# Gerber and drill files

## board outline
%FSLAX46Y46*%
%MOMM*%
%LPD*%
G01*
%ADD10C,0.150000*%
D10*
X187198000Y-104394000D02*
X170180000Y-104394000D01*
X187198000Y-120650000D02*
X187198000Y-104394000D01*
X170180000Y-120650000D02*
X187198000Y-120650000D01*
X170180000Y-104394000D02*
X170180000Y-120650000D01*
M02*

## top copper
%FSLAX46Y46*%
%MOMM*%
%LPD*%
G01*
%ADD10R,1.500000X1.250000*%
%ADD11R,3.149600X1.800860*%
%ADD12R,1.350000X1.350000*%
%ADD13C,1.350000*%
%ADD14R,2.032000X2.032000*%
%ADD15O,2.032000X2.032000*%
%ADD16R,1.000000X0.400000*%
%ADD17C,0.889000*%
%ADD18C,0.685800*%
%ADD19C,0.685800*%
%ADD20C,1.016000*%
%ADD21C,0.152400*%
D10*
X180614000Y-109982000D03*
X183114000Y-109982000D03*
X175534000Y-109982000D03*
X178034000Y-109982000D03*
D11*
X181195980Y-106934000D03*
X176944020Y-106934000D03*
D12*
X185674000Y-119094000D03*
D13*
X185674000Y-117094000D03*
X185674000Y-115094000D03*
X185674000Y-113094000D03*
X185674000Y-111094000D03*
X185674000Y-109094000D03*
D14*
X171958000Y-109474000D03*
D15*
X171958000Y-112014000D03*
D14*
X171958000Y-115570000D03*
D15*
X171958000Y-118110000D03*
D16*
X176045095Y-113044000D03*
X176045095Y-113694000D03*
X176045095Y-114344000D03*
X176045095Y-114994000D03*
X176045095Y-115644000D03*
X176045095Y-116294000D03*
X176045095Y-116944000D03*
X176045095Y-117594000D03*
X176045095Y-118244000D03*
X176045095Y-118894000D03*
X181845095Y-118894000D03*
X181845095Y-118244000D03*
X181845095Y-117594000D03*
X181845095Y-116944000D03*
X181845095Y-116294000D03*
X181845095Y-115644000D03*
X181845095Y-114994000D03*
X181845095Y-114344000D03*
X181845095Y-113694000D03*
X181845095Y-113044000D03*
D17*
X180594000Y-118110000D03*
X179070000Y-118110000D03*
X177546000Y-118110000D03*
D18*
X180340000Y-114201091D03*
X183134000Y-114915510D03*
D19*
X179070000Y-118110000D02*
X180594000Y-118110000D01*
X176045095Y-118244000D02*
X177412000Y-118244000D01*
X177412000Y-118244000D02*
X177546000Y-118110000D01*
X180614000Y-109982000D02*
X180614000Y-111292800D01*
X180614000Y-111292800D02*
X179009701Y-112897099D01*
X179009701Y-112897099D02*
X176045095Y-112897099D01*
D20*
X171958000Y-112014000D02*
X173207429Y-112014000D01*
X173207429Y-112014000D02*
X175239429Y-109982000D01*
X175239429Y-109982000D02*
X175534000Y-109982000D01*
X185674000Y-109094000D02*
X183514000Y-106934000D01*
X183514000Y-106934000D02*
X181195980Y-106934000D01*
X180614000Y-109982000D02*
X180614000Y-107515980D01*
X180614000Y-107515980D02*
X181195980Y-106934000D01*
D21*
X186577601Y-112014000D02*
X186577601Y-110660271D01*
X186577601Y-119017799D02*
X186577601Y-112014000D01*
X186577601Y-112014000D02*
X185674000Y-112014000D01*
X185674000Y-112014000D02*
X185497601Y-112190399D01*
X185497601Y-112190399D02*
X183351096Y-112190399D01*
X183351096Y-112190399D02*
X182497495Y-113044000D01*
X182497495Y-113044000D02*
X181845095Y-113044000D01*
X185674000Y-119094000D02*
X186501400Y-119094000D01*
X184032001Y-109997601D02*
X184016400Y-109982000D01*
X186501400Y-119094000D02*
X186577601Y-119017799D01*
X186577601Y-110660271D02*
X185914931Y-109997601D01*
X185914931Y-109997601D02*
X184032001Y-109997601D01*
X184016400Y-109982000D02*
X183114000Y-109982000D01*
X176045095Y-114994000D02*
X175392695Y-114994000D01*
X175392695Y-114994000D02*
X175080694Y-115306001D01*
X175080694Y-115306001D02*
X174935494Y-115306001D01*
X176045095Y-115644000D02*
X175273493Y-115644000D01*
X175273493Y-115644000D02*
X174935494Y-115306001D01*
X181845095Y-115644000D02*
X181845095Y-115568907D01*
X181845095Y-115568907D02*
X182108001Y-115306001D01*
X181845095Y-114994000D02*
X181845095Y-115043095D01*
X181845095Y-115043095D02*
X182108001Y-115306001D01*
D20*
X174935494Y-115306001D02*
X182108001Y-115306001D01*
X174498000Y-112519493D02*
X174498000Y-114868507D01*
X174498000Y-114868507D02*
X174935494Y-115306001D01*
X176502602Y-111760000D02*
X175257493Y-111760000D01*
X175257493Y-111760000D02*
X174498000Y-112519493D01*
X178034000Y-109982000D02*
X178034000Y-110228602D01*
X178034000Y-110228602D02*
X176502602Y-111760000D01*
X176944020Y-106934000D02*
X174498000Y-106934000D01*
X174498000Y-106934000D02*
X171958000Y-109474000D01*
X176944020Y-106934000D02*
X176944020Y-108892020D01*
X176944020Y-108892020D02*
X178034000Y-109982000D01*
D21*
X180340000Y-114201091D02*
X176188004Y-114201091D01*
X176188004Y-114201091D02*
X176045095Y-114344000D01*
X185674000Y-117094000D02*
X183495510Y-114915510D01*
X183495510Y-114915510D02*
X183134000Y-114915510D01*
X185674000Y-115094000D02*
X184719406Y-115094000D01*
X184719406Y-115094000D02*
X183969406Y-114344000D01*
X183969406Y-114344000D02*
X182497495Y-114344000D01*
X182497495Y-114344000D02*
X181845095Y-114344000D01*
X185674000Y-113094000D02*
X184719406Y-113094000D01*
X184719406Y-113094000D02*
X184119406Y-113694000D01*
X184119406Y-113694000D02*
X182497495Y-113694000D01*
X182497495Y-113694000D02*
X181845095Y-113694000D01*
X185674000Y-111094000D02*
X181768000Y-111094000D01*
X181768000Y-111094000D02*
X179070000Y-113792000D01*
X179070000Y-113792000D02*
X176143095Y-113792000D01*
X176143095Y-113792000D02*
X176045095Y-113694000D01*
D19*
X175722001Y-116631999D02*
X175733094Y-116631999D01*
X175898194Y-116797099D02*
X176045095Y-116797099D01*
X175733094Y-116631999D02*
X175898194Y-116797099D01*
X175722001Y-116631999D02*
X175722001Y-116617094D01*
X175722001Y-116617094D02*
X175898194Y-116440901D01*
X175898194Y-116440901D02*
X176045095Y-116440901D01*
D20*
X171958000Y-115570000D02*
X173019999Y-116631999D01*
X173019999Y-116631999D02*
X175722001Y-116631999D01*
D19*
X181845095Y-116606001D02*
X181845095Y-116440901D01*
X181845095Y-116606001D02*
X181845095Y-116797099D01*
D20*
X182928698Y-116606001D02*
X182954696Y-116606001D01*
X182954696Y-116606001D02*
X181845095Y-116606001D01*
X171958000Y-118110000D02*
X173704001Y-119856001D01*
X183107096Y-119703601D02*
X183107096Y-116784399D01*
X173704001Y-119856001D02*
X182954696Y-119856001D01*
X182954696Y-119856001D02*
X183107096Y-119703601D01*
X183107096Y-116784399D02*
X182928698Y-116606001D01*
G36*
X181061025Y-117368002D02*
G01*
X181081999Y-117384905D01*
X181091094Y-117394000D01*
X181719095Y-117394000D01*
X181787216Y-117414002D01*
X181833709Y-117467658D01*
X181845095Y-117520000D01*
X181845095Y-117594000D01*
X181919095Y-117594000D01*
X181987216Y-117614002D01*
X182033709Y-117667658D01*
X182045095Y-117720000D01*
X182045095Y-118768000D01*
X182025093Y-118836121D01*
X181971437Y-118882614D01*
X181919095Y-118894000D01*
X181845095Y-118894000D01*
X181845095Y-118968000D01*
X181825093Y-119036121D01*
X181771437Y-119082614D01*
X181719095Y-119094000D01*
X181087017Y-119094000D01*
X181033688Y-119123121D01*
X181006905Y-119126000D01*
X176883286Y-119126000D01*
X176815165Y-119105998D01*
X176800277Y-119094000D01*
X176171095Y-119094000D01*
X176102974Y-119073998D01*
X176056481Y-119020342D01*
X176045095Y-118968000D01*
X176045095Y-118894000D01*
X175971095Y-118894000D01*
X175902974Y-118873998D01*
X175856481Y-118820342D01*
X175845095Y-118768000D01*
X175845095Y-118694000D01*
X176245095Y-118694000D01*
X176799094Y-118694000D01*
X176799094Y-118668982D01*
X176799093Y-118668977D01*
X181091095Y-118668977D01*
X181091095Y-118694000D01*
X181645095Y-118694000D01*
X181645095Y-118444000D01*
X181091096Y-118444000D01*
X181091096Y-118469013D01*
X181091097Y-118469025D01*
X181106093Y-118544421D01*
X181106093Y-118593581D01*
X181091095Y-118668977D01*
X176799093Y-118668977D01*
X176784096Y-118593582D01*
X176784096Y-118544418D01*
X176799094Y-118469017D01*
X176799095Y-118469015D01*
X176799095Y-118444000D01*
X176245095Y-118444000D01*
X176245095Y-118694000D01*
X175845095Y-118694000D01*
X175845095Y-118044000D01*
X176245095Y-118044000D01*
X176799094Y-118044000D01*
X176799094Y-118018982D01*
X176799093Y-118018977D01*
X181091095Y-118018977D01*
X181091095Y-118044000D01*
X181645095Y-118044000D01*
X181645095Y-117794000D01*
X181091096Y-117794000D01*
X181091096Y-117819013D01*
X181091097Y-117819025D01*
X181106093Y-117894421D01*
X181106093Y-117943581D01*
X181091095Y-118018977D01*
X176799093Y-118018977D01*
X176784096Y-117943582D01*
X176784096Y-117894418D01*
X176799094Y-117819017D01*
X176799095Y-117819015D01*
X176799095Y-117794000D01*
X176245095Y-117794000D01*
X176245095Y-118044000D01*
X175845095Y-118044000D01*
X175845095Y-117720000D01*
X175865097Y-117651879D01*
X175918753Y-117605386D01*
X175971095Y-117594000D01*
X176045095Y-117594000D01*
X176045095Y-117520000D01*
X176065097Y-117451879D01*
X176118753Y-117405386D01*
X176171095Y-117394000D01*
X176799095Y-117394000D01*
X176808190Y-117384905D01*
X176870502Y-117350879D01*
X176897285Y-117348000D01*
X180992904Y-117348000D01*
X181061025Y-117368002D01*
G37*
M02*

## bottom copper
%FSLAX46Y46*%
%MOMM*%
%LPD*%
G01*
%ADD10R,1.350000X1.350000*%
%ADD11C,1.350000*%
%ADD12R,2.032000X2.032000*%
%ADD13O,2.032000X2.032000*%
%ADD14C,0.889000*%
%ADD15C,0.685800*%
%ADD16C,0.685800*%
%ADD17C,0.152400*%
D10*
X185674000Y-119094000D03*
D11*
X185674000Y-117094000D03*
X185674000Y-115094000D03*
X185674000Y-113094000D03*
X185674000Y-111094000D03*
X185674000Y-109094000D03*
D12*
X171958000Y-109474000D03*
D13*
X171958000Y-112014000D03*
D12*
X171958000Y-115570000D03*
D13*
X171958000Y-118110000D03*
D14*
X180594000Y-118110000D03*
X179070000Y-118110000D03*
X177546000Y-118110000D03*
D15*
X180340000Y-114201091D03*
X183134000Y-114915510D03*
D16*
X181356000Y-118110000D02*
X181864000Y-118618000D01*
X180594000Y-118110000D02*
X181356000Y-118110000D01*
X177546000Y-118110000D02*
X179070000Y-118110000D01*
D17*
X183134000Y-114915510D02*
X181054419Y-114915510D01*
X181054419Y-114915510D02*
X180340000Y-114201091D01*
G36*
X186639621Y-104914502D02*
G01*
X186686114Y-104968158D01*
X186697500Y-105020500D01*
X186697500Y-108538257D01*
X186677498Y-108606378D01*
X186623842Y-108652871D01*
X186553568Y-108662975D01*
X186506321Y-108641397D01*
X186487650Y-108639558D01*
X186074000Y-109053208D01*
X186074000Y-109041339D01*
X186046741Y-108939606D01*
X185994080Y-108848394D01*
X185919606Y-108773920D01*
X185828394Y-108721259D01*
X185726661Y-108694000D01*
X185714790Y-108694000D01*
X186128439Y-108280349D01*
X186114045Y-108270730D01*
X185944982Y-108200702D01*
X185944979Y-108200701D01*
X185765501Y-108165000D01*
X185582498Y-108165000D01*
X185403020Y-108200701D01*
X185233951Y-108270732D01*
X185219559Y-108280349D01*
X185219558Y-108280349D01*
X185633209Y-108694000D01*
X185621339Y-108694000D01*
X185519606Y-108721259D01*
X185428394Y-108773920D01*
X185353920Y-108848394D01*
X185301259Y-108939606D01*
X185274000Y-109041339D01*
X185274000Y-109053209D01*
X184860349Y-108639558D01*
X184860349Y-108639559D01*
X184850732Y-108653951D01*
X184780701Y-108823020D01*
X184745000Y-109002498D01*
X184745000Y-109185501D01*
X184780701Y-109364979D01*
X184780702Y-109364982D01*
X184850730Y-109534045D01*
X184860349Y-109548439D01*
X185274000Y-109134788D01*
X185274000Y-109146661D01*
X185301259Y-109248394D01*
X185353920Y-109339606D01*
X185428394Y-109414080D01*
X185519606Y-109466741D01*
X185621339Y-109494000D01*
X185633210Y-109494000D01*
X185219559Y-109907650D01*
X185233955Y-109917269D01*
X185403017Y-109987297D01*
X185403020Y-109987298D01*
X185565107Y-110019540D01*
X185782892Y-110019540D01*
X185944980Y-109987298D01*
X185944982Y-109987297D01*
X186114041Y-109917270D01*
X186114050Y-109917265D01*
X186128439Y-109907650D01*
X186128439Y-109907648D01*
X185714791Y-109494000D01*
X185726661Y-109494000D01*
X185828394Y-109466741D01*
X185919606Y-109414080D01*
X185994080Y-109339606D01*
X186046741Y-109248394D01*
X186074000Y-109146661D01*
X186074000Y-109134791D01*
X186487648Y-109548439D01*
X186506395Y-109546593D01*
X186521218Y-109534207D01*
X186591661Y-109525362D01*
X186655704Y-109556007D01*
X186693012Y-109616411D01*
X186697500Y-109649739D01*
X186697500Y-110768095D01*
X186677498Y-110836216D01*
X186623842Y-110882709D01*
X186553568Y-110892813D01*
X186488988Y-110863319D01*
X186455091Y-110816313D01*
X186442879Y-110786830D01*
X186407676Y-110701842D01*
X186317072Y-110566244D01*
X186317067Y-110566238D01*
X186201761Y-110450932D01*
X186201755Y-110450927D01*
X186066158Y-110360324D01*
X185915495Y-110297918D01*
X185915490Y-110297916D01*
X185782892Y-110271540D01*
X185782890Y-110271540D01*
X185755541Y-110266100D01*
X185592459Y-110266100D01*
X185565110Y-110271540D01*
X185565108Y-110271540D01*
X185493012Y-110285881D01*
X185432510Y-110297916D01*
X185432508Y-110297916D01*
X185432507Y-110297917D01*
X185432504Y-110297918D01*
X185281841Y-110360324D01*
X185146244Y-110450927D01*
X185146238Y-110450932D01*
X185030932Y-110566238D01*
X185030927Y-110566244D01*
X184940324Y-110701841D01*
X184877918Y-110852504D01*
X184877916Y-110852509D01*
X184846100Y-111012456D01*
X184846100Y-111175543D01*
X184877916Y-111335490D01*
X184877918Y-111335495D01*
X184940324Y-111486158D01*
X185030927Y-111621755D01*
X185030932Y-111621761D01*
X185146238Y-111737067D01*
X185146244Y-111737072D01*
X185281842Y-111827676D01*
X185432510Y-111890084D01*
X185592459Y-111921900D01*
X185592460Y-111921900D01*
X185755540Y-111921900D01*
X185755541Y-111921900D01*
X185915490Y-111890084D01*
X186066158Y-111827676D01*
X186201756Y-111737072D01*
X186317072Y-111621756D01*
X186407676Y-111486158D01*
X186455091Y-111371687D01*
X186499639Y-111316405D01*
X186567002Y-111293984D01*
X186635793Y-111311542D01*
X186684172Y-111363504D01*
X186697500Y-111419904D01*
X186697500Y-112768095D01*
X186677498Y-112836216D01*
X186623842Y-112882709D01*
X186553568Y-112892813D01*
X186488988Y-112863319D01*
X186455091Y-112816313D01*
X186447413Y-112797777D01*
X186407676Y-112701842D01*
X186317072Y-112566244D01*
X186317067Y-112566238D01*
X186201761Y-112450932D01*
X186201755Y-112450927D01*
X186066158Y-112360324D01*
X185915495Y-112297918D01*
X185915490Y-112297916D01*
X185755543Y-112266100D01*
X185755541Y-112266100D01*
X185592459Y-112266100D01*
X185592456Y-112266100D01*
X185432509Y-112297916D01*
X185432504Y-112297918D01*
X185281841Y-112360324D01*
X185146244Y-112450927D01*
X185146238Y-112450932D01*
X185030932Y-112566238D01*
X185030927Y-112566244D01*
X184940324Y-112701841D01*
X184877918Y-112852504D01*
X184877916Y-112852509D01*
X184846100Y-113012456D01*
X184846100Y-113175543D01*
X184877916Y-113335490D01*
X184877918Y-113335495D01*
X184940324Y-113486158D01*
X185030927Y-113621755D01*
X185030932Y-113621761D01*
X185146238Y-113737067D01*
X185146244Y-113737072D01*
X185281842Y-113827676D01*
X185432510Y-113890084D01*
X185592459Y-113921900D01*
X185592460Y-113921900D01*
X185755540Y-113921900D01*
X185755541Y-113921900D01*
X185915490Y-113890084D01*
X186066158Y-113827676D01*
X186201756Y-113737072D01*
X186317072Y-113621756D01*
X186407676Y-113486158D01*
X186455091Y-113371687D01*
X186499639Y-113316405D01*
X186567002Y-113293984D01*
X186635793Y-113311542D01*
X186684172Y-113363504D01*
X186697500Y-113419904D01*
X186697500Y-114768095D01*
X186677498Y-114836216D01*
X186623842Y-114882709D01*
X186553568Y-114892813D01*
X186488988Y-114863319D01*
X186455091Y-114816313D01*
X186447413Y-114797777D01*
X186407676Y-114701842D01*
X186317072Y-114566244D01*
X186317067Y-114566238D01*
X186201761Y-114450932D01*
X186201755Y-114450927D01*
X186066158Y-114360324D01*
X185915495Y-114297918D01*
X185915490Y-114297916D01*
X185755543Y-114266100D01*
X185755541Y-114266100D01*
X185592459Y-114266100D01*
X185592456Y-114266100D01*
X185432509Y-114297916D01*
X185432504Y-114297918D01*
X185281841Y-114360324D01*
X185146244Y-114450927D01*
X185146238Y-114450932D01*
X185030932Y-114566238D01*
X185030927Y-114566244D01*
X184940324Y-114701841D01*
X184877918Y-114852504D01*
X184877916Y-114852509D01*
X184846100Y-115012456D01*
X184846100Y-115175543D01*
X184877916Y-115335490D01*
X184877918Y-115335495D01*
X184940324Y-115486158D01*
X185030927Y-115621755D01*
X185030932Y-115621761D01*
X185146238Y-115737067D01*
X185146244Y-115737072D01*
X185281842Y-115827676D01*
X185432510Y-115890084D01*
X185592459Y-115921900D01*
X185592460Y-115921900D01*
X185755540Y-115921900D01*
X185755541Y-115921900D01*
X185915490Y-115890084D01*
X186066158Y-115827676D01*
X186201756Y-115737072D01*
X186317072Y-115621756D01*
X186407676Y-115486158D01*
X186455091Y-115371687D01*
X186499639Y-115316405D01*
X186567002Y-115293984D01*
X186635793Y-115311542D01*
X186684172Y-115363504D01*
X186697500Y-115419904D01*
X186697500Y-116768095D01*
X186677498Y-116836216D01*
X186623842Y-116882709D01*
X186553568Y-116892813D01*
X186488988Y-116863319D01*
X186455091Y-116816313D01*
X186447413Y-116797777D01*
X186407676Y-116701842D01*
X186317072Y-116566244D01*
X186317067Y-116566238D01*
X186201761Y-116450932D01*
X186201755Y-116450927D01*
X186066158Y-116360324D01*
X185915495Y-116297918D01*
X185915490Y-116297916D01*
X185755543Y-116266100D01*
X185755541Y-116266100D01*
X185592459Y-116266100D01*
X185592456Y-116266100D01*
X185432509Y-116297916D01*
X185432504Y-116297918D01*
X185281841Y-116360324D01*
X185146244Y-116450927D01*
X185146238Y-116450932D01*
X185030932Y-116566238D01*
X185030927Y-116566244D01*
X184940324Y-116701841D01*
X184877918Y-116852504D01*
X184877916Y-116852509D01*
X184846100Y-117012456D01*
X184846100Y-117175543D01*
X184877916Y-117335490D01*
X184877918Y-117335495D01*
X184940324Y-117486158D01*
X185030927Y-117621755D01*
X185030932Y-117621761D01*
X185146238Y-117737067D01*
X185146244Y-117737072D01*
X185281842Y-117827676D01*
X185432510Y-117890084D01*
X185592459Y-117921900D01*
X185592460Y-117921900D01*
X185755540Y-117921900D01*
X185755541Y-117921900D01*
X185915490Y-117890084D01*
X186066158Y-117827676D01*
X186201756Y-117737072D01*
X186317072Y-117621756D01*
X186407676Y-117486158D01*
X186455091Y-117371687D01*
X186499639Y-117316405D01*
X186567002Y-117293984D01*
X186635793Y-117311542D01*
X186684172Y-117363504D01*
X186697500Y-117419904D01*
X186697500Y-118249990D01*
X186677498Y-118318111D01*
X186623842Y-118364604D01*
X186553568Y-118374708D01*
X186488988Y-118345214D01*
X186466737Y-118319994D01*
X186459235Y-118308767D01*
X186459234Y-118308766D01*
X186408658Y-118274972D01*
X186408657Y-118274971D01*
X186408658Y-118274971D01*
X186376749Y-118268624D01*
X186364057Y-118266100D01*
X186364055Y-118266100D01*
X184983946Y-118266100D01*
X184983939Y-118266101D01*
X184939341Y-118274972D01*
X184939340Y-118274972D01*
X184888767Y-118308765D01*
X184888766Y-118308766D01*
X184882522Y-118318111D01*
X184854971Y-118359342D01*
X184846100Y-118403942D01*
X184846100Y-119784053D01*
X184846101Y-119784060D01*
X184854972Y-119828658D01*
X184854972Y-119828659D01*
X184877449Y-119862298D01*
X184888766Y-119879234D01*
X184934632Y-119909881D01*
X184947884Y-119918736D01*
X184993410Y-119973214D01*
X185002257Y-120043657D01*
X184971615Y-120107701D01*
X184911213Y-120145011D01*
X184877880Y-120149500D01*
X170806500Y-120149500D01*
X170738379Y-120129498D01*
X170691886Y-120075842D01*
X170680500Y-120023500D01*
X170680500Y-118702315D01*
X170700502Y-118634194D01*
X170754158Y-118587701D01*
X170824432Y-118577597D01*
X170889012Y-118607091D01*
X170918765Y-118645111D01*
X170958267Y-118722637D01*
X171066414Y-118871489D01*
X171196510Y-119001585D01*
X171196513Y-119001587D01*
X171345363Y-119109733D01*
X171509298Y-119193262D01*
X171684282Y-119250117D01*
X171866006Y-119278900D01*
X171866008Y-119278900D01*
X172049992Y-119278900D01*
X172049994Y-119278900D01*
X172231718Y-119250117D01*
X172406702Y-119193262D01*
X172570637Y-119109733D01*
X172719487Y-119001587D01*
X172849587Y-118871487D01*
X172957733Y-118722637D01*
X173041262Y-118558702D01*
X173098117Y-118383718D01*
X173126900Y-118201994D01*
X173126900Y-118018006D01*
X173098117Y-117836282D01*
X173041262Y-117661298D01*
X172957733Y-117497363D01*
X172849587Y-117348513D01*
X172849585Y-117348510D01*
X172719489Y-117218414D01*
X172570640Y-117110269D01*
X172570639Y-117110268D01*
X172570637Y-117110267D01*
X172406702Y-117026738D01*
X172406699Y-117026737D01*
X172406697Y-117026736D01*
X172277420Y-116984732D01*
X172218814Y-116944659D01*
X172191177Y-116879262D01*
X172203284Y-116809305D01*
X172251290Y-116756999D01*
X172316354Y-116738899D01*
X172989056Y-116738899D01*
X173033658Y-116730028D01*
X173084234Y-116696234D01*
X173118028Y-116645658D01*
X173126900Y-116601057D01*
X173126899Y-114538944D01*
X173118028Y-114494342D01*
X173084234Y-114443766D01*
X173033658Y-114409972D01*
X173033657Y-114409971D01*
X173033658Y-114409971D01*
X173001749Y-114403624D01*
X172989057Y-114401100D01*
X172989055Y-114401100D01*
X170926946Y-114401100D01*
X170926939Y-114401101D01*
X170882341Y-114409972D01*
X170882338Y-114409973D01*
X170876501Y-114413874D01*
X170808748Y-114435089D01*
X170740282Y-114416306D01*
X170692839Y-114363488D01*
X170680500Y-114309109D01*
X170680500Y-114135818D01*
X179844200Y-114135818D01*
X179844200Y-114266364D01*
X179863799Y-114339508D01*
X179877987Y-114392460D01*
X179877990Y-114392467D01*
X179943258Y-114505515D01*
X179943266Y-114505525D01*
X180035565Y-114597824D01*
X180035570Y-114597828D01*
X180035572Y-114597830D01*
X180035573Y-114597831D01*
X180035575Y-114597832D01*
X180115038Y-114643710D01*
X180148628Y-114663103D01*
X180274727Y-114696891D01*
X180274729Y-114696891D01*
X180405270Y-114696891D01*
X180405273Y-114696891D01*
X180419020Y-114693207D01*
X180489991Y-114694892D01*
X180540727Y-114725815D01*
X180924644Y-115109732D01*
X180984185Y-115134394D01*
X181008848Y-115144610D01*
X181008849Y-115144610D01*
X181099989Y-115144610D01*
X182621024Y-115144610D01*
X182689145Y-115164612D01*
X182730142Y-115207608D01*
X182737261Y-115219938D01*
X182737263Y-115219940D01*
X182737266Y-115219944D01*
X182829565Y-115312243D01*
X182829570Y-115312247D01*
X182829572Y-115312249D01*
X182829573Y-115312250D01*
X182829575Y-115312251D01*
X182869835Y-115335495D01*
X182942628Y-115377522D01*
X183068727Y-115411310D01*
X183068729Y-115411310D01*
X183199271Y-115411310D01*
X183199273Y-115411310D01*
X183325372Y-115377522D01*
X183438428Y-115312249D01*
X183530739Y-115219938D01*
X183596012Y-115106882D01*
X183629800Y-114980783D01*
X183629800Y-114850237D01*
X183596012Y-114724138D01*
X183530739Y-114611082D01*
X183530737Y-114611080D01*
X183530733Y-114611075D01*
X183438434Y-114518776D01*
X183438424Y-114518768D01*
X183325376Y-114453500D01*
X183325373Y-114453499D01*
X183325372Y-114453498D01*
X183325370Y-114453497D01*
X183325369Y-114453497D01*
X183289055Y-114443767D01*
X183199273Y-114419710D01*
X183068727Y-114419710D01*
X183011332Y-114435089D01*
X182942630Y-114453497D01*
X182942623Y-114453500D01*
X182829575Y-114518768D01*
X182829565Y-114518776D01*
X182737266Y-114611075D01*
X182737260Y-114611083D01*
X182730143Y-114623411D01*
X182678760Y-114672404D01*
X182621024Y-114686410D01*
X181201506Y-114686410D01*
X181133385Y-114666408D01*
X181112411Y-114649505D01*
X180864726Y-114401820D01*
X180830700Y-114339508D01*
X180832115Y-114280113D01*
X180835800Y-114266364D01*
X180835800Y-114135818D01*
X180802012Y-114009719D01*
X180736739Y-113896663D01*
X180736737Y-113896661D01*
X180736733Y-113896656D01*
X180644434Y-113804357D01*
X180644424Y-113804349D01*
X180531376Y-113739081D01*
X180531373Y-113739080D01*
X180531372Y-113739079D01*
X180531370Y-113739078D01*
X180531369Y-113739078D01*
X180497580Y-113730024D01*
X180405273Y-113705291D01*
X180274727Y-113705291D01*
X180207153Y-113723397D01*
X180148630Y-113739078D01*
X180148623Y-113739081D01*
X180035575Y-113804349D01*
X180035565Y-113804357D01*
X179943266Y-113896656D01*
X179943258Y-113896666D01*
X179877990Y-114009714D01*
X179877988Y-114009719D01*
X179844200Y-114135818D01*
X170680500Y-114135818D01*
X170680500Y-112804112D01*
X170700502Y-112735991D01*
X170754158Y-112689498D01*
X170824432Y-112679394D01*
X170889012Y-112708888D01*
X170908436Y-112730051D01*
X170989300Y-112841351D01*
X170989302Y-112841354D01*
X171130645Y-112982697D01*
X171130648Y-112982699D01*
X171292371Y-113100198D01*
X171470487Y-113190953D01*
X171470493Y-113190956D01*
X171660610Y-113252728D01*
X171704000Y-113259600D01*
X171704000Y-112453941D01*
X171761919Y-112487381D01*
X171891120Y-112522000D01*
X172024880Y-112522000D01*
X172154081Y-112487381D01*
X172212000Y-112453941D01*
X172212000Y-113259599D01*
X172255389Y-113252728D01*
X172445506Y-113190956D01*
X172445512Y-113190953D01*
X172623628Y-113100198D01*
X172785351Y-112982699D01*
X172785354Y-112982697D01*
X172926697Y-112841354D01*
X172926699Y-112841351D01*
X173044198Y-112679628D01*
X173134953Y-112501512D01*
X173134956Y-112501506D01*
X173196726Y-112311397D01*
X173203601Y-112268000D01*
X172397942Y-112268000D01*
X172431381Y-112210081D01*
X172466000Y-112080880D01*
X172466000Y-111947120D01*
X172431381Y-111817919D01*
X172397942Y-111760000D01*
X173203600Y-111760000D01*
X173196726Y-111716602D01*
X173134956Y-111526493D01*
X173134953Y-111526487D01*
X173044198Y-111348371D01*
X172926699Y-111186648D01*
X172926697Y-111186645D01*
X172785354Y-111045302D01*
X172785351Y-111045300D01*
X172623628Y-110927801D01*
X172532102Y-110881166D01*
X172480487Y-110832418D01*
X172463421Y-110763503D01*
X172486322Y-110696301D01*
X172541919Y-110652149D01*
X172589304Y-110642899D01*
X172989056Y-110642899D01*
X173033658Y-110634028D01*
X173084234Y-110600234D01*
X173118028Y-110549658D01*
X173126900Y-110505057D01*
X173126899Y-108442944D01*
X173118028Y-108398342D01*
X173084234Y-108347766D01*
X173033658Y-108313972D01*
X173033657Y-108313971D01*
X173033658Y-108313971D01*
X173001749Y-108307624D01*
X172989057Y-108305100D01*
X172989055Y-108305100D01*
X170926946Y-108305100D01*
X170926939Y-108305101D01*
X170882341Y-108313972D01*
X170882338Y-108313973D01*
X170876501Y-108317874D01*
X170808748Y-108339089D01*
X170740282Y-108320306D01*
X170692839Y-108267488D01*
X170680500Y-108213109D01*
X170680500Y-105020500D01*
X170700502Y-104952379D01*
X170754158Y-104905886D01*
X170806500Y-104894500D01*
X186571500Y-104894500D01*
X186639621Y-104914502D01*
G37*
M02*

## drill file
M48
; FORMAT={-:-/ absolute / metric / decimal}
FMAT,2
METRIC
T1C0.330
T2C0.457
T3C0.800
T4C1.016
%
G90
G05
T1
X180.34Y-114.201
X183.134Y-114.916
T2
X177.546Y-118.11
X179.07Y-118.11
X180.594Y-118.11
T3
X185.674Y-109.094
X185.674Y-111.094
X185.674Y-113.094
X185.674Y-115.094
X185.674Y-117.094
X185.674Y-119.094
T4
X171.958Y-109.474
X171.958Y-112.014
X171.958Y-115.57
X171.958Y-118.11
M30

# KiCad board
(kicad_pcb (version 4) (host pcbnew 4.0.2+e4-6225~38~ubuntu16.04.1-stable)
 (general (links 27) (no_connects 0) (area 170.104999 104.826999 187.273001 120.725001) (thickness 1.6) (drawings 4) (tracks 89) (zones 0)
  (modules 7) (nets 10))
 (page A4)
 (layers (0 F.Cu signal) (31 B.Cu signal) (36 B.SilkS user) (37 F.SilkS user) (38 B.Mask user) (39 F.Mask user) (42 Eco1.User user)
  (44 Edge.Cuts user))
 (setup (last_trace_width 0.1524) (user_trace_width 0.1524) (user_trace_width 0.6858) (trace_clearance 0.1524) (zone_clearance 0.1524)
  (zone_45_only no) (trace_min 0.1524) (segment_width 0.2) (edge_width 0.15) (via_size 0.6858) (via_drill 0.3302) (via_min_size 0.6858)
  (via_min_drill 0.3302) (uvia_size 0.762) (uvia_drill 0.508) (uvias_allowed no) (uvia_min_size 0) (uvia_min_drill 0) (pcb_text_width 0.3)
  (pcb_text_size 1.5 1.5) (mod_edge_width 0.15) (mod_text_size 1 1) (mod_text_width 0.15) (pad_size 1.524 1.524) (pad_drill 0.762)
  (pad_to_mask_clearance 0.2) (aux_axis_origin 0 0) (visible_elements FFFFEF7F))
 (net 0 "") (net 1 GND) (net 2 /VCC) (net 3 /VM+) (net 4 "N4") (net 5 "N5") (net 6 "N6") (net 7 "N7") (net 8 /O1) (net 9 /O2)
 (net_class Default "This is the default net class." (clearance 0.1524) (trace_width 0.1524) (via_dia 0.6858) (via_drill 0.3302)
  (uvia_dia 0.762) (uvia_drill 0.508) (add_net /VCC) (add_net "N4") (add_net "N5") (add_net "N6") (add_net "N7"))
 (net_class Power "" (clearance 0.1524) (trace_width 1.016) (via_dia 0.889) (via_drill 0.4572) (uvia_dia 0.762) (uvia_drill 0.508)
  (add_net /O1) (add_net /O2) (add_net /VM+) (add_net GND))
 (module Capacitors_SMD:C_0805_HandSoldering (layer F.Cu) (at 181.864 109.982)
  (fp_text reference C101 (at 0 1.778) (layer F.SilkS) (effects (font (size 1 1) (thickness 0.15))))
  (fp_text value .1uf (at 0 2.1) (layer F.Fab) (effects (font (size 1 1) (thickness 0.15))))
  (pad 1 smd rect (at -1.25 0) (size 1.5 1.25) (layers F.Cu F.Mask) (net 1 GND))
  (pad 2 smd rect (at 1.25 0) (size 1.5 1.25) (layers F.Cu F.Mask) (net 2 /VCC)))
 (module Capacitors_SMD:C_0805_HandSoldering (layer F.Cu) (at 176.784 109.982)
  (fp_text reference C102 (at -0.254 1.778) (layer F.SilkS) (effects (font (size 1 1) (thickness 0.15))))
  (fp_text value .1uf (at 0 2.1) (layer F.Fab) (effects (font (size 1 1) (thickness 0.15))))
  (pad 1 smd rect (at -1.25 0) (size 1.5 1.25) (layers F.Cu F.Mask) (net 1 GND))
  (pad 2 smd rect (at 1.25 0) (size 1.5 1.25) (layers F.Cu F.Mask) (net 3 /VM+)))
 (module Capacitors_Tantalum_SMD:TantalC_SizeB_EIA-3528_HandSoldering (layer F.Cu) (at 179.07 106.934)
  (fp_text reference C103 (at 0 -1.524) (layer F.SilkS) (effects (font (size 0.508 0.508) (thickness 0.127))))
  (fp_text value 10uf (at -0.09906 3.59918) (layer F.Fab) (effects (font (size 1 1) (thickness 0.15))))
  (pad 2 smd rect (at 2.12598 0) (size 3.1496 1.80086) (layers F.Cu F.Mask) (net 1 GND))
  (pad 1 smd rect (at -2.12598 0) (size 3.1496 1.80086) (layers F.Cu F.Mask) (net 3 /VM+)))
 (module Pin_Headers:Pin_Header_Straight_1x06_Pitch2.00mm (layer F.Cu) (at 185.674 119.094 180)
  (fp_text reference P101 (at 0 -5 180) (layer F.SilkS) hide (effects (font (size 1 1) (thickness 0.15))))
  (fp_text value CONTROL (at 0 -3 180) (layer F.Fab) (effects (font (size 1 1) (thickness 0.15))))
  (pad 1 thru_hole rect (at 0 0 180) (size 1.35 1.35) (drill 0.8) (layers *.Cu *.Mask) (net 2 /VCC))
  (pad 2 thru_hole circle (at 0 2 180) (size 1.35 1.35) (drill 0.8) (layers *.Cu *.Mask) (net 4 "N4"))
  (pad 3 thru_hole circle (at 0 4 180) (size 1.35 1.35) (drill 0.8) (layers *.Cu *.Mask) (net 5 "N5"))
  (pad 4 thru_hole circle (at 0 6 180) (size 1.35 1.35) (drill 0.8) (layers *.Cu *.Mask) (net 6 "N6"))
  (pad 5 thru_hole circle (at 0 8 180) (size 1.35 1.35) (drill 0.8) (layers *.Cu *.Mask) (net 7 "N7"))
  (pad 6 thru_hole circle (at 0 10 180) (size 1.35 1.35) (drill 0.8) (layers *.Cu *.Mask) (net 1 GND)))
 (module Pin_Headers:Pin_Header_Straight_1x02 (layer F.Cu) (at 171.958 109.474)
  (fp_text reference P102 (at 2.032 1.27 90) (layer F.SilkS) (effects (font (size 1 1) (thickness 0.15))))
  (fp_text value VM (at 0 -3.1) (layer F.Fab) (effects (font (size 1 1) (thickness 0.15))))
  (pad 1 thru_hole rect (at 0 0) (size 2.032 2.032) (drill 1.016) (layers *.Cu *.Mask F.SilkS) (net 3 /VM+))
  (pad 2 thru_hole oval (at 0 2.54) (size 2.032 2.032) (drill 1.016) (layers *.Cu *.Mask F.SilkS) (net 1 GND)))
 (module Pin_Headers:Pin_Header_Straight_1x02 (layer F.Cu) (at 171.958 115.57)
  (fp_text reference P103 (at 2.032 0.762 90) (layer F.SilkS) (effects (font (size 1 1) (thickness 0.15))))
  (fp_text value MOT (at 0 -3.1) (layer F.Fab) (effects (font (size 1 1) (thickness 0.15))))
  (pad 1 thru_hole rect (at 0 0) (size 2.032 2.032) (drill 1.016) (layers *.Cu *.Mask F.SilkS) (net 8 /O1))
  (pad 2 thru_hole oval (at 0 2.54) (size 2.032 2.032) (drill 1.016) (layers *.Cu *.Mask F.SilkS) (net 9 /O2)))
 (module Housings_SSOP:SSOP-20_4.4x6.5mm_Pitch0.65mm (layer F.Cu) (at 178.945095 115.969)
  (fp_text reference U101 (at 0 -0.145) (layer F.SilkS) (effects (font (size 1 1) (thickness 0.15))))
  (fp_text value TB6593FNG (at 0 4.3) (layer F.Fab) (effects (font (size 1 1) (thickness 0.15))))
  (pad 1 smd rect (at -2.9 -2.925) (size 1 0.4) (layers F.Cu F.Mask) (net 1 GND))
  (pad 2 smd rect (at -2.9 -2.275) (size 1 0.4) (layers F.Cu F.Mask) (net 7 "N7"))
  (pad 3 smd rect (at -2.9 -1.625) (size 1 0.4) (layers F.Cu F.Mask) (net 4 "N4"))
  (pad 4 smd rect (at -2.9 -0.975) (size 1 0.4) (layers F.Cu F.Mask) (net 3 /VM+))
  (pad 5 smd rect (at -2.9 -0.325) (size 1 0.4) (layers F.Cu F.Mask) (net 3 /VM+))
  (pad 6 smd rect (at -2.9 0.325) (size 1 0.4) (layers F.Cu F.Mask) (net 8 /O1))
  (pad 7 smd rect (at -2.9 0.975) (size 1 0.4) (layers F.Cu F.Mask) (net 8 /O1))
  (pad 8 smd rect (at -2.9 1.625) (size 1 0.4) (layers F.Cu F.Mask) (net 1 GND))
  (pad 9 smd rect (at -2.9 2.275) (size 1 0.4) (layers F.Cu F.Mask) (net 1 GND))
  (pad 10 smd rect (at -2.9 2.925) (size 1 0.4) (layers F.Cu F.Mask) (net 1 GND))
  (pad 11 smd rect (at 2.9 2.925) (size 1 0.4) (layers F.Cu F.Mask) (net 1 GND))
  (pad 12 smd rect (at 2.9 2.275) (size 1 0.4) (layers F.Cu F.Mask) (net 1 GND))
  (pad 13 smd rect (at 2.9 1.625) (size 1 0.4) (layers F.Cu F.Mask) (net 1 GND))
  (pad 14 smd rect (at 2.9 0.975) (size 1 0.4) (layers F.Cu F.Mask) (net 9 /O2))
  (pad 15 smd rect (at 2.9 0.325) (size 1 0.4) (layers F.Cu F.Mask) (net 9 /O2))
  (pad 16 smd rect (at 2.9 -0.325) (size 1 0.4) (layers F.Cu F.Mask) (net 3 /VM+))
  (pad 17 smd rect (at 2.9 -0.975) (size 1 0.4) (layers F.Cu F.Mask) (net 3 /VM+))
  (pad 18 smd rect (at 2.9 -1.625) (size 1 0.4) (layers F.Cu F.Mask) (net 5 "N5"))
  (pad 19 smd rect (at 2.9 -2.275) (size 1 0.4) (layers F.Cu F.Mask) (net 6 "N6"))
  (pad 20 smd rect (at 2.9 -2.925) (size 1 0.4) (layers F.Cu F.Mask) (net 2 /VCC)))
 (gr_line (start 187.198 104.394) (end 170.18 104.394) (layer Edge.Cuts) (width 0.15))
 (gr_line (start 187.198 120.65) (end 187.198 104.394) (layer Edge.Cuts) (width 0.15))
 (gr_line (start 170.18 120.65) (end 187.198 120.65) (layer Edge.Cuts) (width 0.15))
 (gr_line (start 170.18 104.394) (end 170.18 120.65) (layer Edge.Cuts) (width 0.15))
 (segment (start 181.356 118.11) (end 181.864 118.618) (width 0.6858) (layer B.Cu) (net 1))
 (segment (start 180.594 118.11) (end 181.356 118.11) (width 0.6858) (layer B.Cu) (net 1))
 (segment (start 179.07 118.11) (end 180.594 118.11) (width 0.6858) (layer F.Cu) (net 1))
 (via (at 180.594 118.11) (size 0.889) (drill 0.4572) (layers F.Cu B.Cu) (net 1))
 (via (at 179.07 118.11) (size 0.889) (drill 0.4572) (layers F.Cu B.Cu) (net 1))
 (segment (start 177.546 118.11) (end 179.07 118.11) (width 0.6858) (layer B.Cu) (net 1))
 (segment (start 176.045095 118.244) (end 177.412 118.244) (width 0.6858) (layer F.Cu) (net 1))
 (segment (start 177.412 118.244) (end 177.546 118.11) (width 0.6858) (layer F.Cu) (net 1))
 (via (at 177.546 118.11) (size 0.889) (drill 0.4572) (layers F.Cu B.Cu) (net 1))
 (segment (start 180.614 109.982) (end 180.614 111.2928) (width 0.6858) (layer F.Cu) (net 1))
 (segment (start 180.614 111.2928) (end 179.009701 112.897099) (width 0.6858) (layer F.Cu) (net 1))
 (segment (start 179.009701 112.897099) (end 176.045095 112.897099) (width 0.6858) (layer F.Cu) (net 1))
 (segment (start 171.958 112.014) (end 173.207429 112.014) (width 1.016) (layer F.Cu) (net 1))
 (segment (start 173.207429 112.014) (end 175.239429 109.982) (width 1.016) (layer F.Cu) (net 1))
 (segment (start 175.239429 109.982) (end 175.534 109.982) (width 1.016) (layer F.Cu) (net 1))
 (segment (start 185.674 109.094) (end 183.514 106.934) (width 1.016) (layer F.Cu) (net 1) (status 10))
 (segment (start 183.514 106.934) (end 181.19598 106.934) (width 1.016) (layer F.Cu) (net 1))
 (segment (start 180.614 109.982) (end 180.614 107.51598) (width 1.016) (layer F.Cu) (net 1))
 (segment (start 180.614 107.51598) (end 181.19598 106.934) (width 1.016) (layer F.Cu) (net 1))
 (segment (start 186.577601 112.014) (end 186.577601 110.660271) (width 0.1524) (layer F.Cu) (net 2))
 (segment (start 186.577601 119.017799) (end 186.577601 112.014) (width 0.1524) (layer F.Cu) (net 2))
 (segment (start 186.577601 112.014) (end 185.674 112.014) (width 0.1524) (layer F.Cu) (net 2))
 (segment (start 185.674 112.014) (end 185.497601 112.190399) (width 0.1524) (layer F.Cu) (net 2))
 (segment (start 185.497601 112.190399) (end 183.351096 112.190399) (width 0.1524) (layer F.Cu) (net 2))
 (segment (start 183.351096 112.190399) (end 182.497495 113.044) (width 0.1524) (layer F.Cu) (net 2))
 (segment (start 182.497495 113.044) (end 181.845095 113.044) (width 0.1524) (layer F.Cu) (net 2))
 (segment (start 185.674 119.094) (end 186.5014 119.094) (width 0.1524) (layer F.Cu) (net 2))
 (segment (start 184.032001 109.997601) (end 184.0164 109.982) (width 0.1524) (layer F.Cu) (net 2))
 (segment (start 186.5014 119.094) (end 186.577601 119.017799) (width 0.1524) (layer F.Cu) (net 2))
 (segment (start 186.577601 110.660271) (end 185.914931 109.997601) (width 0.1524) (layer F.Cu) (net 2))
 (segment (start 185.914931 109.997601) (end 184.032001 109.997601) (width 0.1524) (layer F.Cu) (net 2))
 (segment (start 184.0164 109.982) (end 183.114 109.982) (width 0.1524) (layer F.Cu) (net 2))
 (segment (start 176.045095 114.994) (end 175.392695 114.994) (width 0.1524) (layer F.Cu) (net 3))
 (segment (start 175.392695 114.994) (end 175.080694 115.306001) (width 0.1524) (layer F.Cu) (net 3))
 (segment (start 175.080694 115.306001) (end 174.935494 115.306001) (width 0.1524) (layer F.Cu) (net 3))
 (segment (start 176.045095 115.644) (end 175.273493 115.644) (width 0.1524) (layer F.Cu) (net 3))
 (segment (start 175.273493 115.644) (end 174.935494 115.306001) (width 0.1524) (layer F.Cu) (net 3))
 (segment (start 181.845095 115.644) (end 181.845095 115.568907) (width 0.1524) (layer F.Cu) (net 3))
 (segment (start 181.845095 115.568907) (end 182.108001 115.306001) (width 0.1524) (layer F.Cu) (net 3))
 (segment (start 181.845095 114.994) (end 181.845095 115.043095) (width 0.1524) (layer F.Cu) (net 3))
 (segment (start 181.845095 115.043095) (end 182.108001 115.306001) (width 0.1524) (layer F.Cu) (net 3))
 (segment (start 174.935494 115.306001) (end 182.108001 115.306001) (width 1.016) (layer F.Cu) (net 3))
 (segment (start 174.498 112.519493) (end 174.498 114.868507) (width 1.016) (layer F.Cu) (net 3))
 (segment (start 174.498 114.868507) (end 174.935494 115.306001) (width 1.016) (layer F.Cu) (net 3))
 (segment (start 176.502602 111.76) (end 175.257493 111.76) (width 1.016) (layer F.Cu) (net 3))
 (segment (start 175.257493 111.76) (end 174.498 112.519493) (width 1.016) (layer F.Cu) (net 3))
 (segment (start 178.034 109.982) (end 178.034 110.228602) (width 1.016) (layer F.Cu) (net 3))
 (segment (start 178.034 110.228602) (end 176.502602 111.76) (width 1.016) (layer F.Cu) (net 3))
 (segment (start 176.94402 106.934) (end 174.498 106.934) (width 1.016) (layer F.Cu) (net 3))
 (segment (start 174.498 106.934) (end 171.958 109.474) (width 1.016) (layer F.Cu) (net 3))
 (segment (start 176.94402 106.934) (end 176.94402 108.89202) (width 1.016) (layer F.Cu) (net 3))
 (segment (start 176.94402 108.89202) (end 178.034 109.982) (width 1.016) (layer F.Cu) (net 3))
 (segment (start 180.34 114.201091) (end 176.188004 114.201091) (width 0.1524) (layer F.Cu) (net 4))
 (segment (start 176.188004 114.201091) (end 176.045095 114.344) (width 0.1524) (layer F.Cu) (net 4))
 (segment (start 183.134 114.91551) (end 181.054419 114.91551) (width 0.1524) (layer B.Cu) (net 4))
 (segment (start 181.054419 114.91551) (end 180.34 114.201091) (width 0.1524) (layer B.Cu) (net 4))
 (via (at 180.34 114.201091) (size 0.6858) (drill 0.3302) (layers F.Cu B.Cu) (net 4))
 (segment (start 185.674 117.094) (end 183.49551 114.91551) (width 0.1524) (layer F.Cu) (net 4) (status 10))
 (segment (start 183.49551 114.91551) (end 183.134 114.91551) (width 0.1524) (layer F.Cu) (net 4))
 (via (at 183.134 114.91551) (size 0.6858) (drill 0.3302) (layers F.Cu B.Cu) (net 4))
 (segment (start 185.674 115.094) (end 184.719406 115.094) (width 0.1524) (layer F.Cu) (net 5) (status 10))
 (segment (start 184.719406 115.094) (end 183.969406 114.344) (width 0.1524) (layer F.Cu) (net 5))
 (segment (start 183.969406 114.344) (end 182.497495 114.344) (width 0.1524) (layer F.Cu) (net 5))
 (segment (start 182.497495 114.344) (end 181.845095 114.344) (width 0.1524) (layer F.Cu) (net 5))
 (segment (start 185.674 113.094) (end 184.719406 113.094) (width 0.1524) (layer F.Cu) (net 6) (status 10))
 (segment (start 184.719406 113.094) (end 184.119406 113.694) (width 0.1524) (layer F.Cu) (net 6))
 (segment (start 184.119406 113.694) (end 182.497495 113.694) (width 0.1524) (layer F.Cu) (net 6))
 (segment (start 182.497495 113.694) (end 181.845095 113.694) (width 0.1524) (layer F.Cu) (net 6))
 (segment (start 185.674 111.094) (end 181.768 111.094) (width 0.1524) (layer F.Cu) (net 7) (status 10))
 (segment (start 181.768 111.094) (end 179.07 113.792) (width 0.1524) (layer F.Cu) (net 7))
 (segment (start 179.07 113.792) (end 176.143095 113.792) (width 0.1524) (layer F.Cu) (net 7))
 (segment (start 176.143095 113.792) (end 176.045095 113.694) (width 0.1524) (layer F.Cu) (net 7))
 (segment (start 175.722001 116.631999) (end 175.733094 116.631999) (width 0.6858) (layer F.Cu) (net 8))
 (segment (start 175.898194 116.797099) (end 176.045095 116.797099) (width 0.6858) (layer F.Cu) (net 8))
 (segment (start 175.733094 116.631999) (end 175.898194 116.797099) (width 0.6858) (layer F.Cu) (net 8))
 (segment (start 175.722001 116.631999) (end 175.722001 116.617094) (width 0.6858) (layer F.Cu) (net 8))
 (segment (start 175.722001 116.617094) (end 175.898194 116.440901) (width 0.6858) (layer F.Cu) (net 8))
 (segment (start 175.898194 116.440901) (end 176.045095 116.440901) (width 0.6858) (layer F.Cu) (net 8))
 (segment (start 171.958 115.57) (end 173.019999 116.631999) (width 1.016) (layer F.Cu) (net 8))
 (segment (start 173.019999 116.631999) (end 175.722001 116.631999) (width 1.016) (layer F.Cu) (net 8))
 (segment (start 181.845095 116.606001) (end 181.845095 116.440901) (width 0.6858) (layer F.Cu) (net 9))
 (segment (start 181.845095 116.606001) (end 181.845095 116.797099) (width 0.6858) (layer F.Cu) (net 9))
 (segment (start 182.928698 116.606001) (end 182.954696 116.606001) (width 1.016) (layer F.Cu) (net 9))
 (segment (start 182.954696 116.606001) (end 181.845095 116.606001) (width 1.016) (layer F.Cu) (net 9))
 (segment (start 171.958 118.11) (end 173.704001 119.856001) (width 1.016) (layer F.Cu) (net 9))
 (segment (start 183.107096 119.703601) (end 183.107096 116.784399) (width 1.016) (layer F.Cu) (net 9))
 (segment (start 173.704001 119.856001) (end 182.954696 119.856001) (width 1.016) (layer F.Cu) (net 9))
 (segment (start 182.954696 119.856001) (end 183.107096 119.703601) (width 1.016) (layer F.Cu) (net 9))
 (segment (start 183.107096 116.784399) (end 182.928698 116.606001) (width 1.016) (layer F.Cu) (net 9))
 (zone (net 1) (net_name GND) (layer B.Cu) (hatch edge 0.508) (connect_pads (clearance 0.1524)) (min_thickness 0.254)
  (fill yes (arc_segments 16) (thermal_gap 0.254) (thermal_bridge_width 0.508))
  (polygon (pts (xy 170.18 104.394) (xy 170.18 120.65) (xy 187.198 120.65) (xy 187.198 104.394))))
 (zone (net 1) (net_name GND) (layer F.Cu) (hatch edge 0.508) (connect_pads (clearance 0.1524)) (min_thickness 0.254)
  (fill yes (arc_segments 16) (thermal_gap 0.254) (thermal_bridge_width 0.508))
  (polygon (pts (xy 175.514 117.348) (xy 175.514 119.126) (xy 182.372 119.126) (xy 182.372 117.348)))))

